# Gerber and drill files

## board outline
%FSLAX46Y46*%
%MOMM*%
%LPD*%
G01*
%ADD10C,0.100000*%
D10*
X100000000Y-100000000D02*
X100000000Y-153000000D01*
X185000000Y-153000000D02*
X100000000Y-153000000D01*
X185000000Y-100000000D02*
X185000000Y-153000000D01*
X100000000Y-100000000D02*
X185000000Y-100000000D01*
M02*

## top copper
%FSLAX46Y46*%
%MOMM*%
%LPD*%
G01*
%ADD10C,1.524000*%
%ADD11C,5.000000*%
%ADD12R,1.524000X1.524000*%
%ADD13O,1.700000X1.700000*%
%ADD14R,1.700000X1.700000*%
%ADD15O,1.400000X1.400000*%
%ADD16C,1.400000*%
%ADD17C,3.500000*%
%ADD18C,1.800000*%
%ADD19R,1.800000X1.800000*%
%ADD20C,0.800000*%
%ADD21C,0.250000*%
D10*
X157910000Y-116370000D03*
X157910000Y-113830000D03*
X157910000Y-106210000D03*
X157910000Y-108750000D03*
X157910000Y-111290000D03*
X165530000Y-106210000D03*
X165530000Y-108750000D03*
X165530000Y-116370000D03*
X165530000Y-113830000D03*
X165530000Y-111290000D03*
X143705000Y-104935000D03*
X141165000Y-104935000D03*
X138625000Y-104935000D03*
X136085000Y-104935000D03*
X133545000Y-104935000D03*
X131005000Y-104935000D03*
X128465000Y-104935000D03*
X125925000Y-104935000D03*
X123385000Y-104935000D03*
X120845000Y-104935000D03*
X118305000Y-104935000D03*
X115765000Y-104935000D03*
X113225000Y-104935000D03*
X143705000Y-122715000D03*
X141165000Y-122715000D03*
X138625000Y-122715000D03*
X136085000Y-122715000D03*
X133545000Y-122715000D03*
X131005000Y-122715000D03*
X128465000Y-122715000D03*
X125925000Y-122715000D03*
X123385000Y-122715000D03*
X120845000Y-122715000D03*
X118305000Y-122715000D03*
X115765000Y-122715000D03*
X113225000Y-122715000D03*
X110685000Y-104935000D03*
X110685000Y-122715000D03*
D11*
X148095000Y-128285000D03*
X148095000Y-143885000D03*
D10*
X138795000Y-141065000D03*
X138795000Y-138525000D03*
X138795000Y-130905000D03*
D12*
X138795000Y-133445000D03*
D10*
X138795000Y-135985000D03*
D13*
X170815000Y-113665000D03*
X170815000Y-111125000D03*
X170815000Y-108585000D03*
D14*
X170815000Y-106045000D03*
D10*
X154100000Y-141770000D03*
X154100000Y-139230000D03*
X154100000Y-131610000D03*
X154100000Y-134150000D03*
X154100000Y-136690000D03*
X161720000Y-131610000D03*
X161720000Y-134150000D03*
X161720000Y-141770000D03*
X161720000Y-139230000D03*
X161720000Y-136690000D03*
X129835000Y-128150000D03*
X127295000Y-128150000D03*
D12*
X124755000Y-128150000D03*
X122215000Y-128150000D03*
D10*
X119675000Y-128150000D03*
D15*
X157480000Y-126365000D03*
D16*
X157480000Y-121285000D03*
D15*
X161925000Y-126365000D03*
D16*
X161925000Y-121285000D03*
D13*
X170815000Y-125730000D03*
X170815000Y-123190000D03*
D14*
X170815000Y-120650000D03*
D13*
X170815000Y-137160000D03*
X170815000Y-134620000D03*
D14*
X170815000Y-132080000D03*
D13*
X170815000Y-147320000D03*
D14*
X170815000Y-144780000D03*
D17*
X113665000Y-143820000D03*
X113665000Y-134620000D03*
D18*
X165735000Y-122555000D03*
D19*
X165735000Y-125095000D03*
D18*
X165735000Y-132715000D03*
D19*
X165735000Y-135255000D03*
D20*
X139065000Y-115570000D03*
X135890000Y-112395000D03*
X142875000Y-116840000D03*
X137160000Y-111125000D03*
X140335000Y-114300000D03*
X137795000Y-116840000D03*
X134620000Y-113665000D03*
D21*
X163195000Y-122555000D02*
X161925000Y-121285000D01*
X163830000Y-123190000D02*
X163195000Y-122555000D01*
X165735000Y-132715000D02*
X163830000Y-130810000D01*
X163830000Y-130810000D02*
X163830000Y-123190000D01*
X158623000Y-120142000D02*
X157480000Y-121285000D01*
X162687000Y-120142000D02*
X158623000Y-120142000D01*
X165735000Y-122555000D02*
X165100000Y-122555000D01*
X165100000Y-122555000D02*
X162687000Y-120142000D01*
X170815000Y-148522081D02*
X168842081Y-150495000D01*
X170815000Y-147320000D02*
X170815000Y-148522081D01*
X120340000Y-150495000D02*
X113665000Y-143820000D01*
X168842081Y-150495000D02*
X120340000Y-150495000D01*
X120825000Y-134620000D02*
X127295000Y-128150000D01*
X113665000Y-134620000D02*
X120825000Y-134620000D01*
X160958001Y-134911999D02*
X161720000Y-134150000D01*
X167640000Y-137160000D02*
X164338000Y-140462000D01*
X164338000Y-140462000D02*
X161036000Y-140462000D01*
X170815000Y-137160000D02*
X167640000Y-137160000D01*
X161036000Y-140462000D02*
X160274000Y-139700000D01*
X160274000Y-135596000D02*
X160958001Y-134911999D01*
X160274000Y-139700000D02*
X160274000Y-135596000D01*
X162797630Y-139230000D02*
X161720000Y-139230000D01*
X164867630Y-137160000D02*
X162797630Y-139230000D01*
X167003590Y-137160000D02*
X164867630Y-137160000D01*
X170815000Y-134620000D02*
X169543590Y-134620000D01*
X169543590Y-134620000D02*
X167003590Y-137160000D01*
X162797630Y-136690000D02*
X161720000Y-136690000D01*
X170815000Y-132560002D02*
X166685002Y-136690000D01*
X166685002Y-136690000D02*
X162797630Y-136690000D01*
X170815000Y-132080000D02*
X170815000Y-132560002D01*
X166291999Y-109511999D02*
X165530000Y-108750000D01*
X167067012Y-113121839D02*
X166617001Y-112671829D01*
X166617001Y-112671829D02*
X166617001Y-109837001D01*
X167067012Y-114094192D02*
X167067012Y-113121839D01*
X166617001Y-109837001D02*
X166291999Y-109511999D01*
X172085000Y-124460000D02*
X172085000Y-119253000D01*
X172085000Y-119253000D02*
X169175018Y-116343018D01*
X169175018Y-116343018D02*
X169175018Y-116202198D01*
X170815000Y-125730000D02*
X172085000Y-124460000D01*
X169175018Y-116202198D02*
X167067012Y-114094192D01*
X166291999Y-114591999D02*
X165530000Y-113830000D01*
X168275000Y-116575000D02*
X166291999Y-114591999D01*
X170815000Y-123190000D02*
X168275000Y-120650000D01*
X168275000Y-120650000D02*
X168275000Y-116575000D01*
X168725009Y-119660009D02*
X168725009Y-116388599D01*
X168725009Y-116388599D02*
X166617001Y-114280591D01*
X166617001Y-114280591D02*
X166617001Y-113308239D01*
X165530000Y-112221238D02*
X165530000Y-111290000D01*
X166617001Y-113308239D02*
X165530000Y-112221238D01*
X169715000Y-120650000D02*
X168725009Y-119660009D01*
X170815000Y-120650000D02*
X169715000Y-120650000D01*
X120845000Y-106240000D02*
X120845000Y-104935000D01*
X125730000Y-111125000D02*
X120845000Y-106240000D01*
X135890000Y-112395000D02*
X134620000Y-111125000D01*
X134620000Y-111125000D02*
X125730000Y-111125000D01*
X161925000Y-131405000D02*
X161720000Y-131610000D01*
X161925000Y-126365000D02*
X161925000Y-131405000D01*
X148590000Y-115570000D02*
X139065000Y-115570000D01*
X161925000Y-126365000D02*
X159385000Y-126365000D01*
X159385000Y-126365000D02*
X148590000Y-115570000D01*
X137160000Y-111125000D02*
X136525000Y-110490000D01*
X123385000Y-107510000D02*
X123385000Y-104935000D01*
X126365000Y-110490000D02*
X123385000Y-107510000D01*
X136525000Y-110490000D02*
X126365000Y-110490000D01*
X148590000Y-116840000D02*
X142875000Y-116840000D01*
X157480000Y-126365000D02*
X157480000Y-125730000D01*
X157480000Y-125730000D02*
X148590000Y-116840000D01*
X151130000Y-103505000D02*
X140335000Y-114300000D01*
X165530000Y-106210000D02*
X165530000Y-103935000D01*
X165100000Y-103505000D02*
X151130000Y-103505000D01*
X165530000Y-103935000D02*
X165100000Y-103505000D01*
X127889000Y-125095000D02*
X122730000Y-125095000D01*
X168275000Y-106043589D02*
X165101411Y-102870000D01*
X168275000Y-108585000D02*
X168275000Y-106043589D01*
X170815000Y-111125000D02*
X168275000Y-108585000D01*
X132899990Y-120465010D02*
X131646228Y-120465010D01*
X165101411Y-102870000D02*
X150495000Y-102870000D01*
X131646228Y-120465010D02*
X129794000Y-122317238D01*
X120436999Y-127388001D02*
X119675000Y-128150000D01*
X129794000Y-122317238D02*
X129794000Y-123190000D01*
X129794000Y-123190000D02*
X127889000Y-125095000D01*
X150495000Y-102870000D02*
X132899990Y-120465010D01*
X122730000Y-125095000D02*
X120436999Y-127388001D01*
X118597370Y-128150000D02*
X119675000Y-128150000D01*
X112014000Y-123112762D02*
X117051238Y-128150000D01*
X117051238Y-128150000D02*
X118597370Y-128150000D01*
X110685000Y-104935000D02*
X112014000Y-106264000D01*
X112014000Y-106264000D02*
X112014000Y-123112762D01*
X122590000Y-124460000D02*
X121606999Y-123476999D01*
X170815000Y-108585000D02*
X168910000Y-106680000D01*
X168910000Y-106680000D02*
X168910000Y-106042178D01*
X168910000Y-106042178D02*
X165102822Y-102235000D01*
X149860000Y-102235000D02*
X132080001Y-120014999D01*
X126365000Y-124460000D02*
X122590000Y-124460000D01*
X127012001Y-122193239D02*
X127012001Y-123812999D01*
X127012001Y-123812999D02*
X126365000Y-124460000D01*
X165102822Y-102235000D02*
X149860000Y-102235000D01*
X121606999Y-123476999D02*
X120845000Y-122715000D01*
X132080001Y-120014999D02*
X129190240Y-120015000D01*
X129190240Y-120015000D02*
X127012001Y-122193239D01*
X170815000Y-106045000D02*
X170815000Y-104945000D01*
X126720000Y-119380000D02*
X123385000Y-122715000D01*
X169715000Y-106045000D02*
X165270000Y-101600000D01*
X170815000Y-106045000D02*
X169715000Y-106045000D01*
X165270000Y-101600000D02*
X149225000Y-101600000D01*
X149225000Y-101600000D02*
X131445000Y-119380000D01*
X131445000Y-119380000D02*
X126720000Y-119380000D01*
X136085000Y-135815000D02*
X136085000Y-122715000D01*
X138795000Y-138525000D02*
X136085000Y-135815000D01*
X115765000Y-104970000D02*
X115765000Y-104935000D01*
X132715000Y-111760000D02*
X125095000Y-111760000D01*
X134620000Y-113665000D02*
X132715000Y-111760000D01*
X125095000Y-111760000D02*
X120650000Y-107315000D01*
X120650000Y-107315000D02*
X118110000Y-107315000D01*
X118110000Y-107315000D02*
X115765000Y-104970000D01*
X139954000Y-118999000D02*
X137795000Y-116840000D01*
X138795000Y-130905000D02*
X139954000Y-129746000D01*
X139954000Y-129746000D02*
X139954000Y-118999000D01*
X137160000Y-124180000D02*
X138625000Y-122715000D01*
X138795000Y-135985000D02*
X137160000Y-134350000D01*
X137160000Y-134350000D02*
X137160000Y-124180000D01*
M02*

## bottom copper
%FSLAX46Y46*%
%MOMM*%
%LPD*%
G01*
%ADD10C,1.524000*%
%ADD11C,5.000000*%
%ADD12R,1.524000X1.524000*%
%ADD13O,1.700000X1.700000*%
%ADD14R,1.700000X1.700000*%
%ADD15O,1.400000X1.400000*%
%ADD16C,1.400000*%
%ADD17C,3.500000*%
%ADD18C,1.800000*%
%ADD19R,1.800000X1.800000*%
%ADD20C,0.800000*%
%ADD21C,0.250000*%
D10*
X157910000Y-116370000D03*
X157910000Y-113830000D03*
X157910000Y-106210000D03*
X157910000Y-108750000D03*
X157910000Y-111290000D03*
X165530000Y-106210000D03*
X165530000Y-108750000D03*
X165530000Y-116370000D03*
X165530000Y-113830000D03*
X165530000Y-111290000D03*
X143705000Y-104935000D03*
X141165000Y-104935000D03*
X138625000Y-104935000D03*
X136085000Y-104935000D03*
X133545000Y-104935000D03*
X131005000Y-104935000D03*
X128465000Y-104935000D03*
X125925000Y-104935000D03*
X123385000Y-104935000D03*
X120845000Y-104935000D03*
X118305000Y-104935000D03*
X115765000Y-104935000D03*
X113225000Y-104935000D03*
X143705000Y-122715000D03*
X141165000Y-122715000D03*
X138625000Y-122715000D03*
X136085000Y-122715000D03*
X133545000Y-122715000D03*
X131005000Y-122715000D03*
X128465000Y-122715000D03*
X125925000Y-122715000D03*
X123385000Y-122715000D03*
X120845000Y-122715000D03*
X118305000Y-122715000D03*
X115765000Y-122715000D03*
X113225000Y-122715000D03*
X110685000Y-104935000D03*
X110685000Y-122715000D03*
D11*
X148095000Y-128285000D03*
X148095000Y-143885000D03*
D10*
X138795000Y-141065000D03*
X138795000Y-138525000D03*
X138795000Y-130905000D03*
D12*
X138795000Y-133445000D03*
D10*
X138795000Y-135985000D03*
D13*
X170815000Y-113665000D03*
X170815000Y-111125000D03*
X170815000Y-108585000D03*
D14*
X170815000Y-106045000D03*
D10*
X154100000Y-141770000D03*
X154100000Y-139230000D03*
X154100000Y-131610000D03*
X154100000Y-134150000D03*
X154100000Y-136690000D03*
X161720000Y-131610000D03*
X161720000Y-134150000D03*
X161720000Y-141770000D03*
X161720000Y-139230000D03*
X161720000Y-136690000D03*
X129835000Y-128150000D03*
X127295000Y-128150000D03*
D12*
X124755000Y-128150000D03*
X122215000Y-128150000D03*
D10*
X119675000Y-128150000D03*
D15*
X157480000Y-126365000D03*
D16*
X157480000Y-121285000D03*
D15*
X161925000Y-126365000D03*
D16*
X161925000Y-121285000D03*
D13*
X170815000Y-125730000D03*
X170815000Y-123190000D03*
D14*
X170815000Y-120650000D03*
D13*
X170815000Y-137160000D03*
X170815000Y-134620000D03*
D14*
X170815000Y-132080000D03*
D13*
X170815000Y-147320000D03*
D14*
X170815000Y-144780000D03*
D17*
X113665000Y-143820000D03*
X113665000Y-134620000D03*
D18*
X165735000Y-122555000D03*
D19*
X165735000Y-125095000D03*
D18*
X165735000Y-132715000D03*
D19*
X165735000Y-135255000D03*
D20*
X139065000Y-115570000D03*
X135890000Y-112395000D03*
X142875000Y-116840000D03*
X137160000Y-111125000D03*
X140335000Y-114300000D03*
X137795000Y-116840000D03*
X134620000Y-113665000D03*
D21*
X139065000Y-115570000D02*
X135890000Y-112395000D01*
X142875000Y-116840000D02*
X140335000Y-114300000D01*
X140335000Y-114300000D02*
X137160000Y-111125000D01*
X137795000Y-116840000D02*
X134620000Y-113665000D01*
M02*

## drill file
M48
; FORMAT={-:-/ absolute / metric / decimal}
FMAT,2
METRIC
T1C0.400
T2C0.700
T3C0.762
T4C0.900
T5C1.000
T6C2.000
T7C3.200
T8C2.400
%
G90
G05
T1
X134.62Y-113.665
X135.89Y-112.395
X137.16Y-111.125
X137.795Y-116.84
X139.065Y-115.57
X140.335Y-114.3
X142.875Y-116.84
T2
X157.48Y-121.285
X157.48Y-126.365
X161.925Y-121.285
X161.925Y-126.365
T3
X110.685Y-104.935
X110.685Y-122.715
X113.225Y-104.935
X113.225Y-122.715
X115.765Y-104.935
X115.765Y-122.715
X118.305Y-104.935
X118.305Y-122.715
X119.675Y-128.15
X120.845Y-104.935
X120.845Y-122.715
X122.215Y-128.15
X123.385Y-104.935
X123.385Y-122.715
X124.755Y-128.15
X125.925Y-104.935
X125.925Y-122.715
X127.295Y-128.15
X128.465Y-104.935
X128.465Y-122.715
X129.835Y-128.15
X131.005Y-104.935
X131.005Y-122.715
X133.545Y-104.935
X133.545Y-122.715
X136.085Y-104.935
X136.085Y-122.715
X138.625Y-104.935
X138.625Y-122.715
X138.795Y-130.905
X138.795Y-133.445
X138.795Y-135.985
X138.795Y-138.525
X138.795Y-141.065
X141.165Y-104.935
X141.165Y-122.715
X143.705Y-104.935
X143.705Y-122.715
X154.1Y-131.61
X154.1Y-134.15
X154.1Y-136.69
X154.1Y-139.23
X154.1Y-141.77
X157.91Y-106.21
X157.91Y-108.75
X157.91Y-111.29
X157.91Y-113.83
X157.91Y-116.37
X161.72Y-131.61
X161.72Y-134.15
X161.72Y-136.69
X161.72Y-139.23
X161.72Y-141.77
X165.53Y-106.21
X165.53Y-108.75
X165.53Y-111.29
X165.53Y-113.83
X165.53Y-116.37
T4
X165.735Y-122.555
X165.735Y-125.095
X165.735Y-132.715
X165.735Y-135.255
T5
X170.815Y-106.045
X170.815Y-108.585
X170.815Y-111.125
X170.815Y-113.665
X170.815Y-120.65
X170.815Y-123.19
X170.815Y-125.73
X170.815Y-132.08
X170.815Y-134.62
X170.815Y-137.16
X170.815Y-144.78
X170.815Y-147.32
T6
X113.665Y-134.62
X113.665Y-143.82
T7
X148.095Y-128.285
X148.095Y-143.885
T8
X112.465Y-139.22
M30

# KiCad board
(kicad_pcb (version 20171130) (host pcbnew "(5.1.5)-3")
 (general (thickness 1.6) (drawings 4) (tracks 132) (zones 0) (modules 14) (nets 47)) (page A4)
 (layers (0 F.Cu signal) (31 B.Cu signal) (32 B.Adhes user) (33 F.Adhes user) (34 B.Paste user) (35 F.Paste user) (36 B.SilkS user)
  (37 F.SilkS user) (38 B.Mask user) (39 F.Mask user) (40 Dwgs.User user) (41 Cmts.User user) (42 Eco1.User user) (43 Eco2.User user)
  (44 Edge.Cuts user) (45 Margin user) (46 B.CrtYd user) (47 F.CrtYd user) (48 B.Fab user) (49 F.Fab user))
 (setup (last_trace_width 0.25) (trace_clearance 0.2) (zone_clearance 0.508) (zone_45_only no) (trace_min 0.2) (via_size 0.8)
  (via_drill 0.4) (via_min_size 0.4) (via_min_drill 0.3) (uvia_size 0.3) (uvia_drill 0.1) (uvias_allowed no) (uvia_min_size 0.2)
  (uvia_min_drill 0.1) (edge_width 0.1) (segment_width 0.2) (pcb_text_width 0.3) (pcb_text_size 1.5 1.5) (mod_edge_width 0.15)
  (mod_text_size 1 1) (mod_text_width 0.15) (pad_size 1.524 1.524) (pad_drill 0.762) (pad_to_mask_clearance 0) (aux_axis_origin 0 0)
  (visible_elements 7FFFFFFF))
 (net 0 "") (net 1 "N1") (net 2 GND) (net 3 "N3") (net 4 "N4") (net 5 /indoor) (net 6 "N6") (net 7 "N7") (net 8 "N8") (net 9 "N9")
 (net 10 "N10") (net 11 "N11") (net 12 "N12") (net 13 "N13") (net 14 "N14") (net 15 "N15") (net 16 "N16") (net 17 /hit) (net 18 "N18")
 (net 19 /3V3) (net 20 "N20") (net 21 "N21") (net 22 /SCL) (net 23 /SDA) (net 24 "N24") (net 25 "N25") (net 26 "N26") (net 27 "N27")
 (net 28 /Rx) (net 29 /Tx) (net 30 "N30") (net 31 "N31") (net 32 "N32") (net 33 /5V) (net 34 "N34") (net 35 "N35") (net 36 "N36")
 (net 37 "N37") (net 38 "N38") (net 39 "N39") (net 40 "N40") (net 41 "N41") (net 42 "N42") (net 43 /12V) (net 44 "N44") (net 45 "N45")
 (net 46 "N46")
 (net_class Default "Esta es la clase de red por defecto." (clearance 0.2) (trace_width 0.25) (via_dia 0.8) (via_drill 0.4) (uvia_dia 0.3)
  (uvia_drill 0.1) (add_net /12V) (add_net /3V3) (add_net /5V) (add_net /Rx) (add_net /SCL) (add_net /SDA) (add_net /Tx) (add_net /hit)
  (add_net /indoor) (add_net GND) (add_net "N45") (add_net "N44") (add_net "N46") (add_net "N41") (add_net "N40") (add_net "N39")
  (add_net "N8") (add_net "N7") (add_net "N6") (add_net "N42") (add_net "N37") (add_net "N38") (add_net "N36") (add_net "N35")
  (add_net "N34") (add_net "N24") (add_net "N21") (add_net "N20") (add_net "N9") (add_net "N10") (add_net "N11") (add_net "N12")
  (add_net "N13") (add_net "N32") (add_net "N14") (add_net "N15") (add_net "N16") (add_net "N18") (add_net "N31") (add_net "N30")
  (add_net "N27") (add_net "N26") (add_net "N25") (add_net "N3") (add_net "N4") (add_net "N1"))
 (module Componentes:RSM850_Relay (layer F.Cu) (at 166.37 104.14 270)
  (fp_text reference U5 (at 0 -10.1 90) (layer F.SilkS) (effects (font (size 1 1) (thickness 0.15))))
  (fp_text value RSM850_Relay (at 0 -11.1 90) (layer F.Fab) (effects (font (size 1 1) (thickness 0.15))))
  (pad "" thru_hole circle (at 12.23 8.46 270) (size 1.524 1.524) (drill 0.762) (layers *.Cu *.Mask))
  (pad 8 thru_hole circle (at 9.69 8.46 270) (size 1.524 1.524) (drill 0.762) (layers *.Cu *.Mask) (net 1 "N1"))
  (pad 2 thru_hole circle (at 2.07 8.46 270) (size 1.524 1.524) (drill 0.762) (layers *.Cu *.Mask) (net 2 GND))
  (pad 6 thru_hole circle (at 4.61 8.46 270) (size 1.524 1.524) (drill 0.762) (layers *.Cu *.Mask) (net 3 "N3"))
  (pad 7 thru_hole circle (at 7.15 8.46 270) (size 1.524 1.524) (drill 0.762) (layers *.Cu *.Mask) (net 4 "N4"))
  (pad 1 thru_hole circle (at 2.07 0.84 270) (size 1.524 1.524) (drill 0.762) (layers *.Cu *.Mask) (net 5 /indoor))
  (pad 3 thru_hole circle (at 4.61 0.84 270) (size 1.524 1.524) (drill 0.762) (layers *.Cu *.Mask) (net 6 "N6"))
  (pad "" thru_hole circle (at 12.23 0.84 270) (size 1.524 1.524) (drill 0.762) (layers *.Cu *.Mask))
  (pad 5 thru_hole circle (at 9.69 0.84 270) (size 1.524 1.524) (drill 0.762) (layers *.Cu *.Mask) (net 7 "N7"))
  (pad 4 thru_hole circle (at 7.15 0.84 270) (size 1.524 1.524) (drill 0.762) (layers *.Cu *.Mask) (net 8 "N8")))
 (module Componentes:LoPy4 (layer F.Cu) (at 100.965 123.825 90)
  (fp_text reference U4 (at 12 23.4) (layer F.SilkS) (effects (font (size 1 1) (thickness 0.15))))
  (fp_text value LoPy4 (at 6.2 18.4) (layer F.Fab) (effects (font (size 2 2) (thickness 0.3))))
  (pad 15 thru_hole circle (at 18.89 42.74 90) (size 1.524 1.524) (drill 0.762) (layers *.Cu *.Mask) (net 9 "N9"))
  (pad 16 thru_hole circle (at 18.89 40.2 90) (size 1.524 1.524) (drill 0.762) (layers *.Cu *.Mask) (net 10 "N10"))
  (pad 17 thru_hole circle (at 18.89 37.66 90) (size 1.524 1.524) (drill 0.762) (layers *.Cu *.Mask) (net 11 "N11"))
  (pad 18 thru_hole circle (at 18.89 35.12 90) (size 1.524 1.524) (drill 0.762) (layers *.Cu *.Mask) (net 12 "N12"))
  (pad 19 thru_hole circle (at 18.89 32.58 90) (size 1.524 1.524) (drill 0.762) (layers *.Cu *.Mask) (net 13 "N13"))
  (pad 20 thru_hole circle (at 18.89 30.04 90) (size 1.524 1.524) (drill 0.762) (layers *.Cu *.Mask) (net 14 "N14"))
  (pad 21 thru_hole circle (at 18.89 27.5 90) (size 1.524 1.524) (drill 0.762) (layers *.Cu *.Mask) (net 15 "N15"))
  (pad 22 thru_hole circle (at 18.89 24.96 90) (size 1.524 1.524) (drill 0.762) (layers *.Cu *.Mask) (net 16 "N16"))
  (pad 23 thru_hole circle (at 18.89 22.42 90) (size 1.524 1.524) (drill 0.762) (layers *.Cu *.Mask) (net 5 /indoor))
  (pad 24 thru_hole circle (at 18.89 19.88 90) (size 1.524 1.524) (drill 0.762) (layers *.Cu *.Mask) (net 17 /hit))
  (pad 25 thru_hole circle (at 18.89 17.34 90) (size 1.524 1.524) (drill 0.762) (layers *.Cu *.Mask) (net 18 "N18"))
  (pad 26 thru_hole circle (at 18.89 14.8 90) (size 1.524 1.524) (drill 0.762) (layers *.Cu *.Mask) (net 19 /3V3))
  (pad 27 thru_hole circle (at 18.89 12.26 90) (size 1.524 1.524) (drill 0.762) (layers *.Cu *.Mask) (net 2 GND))
  (pad 14 thru_hole circle (at 1.11 42.74 90) (size 1.524 1.524) (drill 0.762) (layers *.Cu *.Mask) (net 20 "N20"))
  (pad 13 thru_hole circle (at 1.11 40.2 90) (size 1.524 1.524) (drill 0.762) (layers *.Cu *.Mask) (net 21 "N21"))
  (pad 12 thru_hole circle (at 1.11 37.66 90) (size 1.524 1.524) (drill 0.762) (layers *.Cu *.Mask) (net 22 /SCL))
  (pad 11 thru_hole circle (at 1.11 35.12 90) (size 1.524 1.524) (drill 0.762) (layers *.Cu *.Mask) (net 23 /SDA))
  (pad 10 thru_hole circle (at 1.11 32.58 90) (size 1.524 1.524) (drill 0.762) (layers *.Cu *.Mask) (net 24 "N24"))
  (pad 9 thru_hole circle (at 1.11 30.04 90) (size 1.524 1.524) (drill 0.762) (layers *.Cu *.Mask) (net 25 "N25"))
  (pad 8 thru_hole circle (at 1.11 27.5 90) (size 1.524 1.524) (drill 0.762) (layers *.Cu *.Mask) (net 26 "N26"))
  (pad 7 thru_hole circle (at 1.11 24.96 90) (size 1.524 1.524) (drill 0.762) (layers *.Cu *.Mask) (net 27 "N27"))
  (pad 6 thru_hole circle (at 1.11 22.42 90) (size 1.524 1.524) (drill 0.762) (layers *.Cu *.Mask) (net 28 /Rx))
  (pad 5 thru_hole circle (at 1.11 19.88 90) (size 1.524 1.524) (drill 0.762) (layers *.Cu *.Mask) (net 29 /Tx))
  (pad 4 thru_hole circle (at 1.11 17.34 90) (size 1.524 1.524) (drill 0.762) (layers *.Cu *.Mask) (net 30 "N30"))
  (pad 3 thru_hole circle (at 1.11 14.8 90) (size 1.524 1.524) (drill 0.762) (layers *.Cu *.Mask) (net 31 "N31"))
  (pad 2 thru_hole circle (at 1.11 12.26 90) (size 1.524 1.524) (drill 0.762) (layers *.Cu *.Mask) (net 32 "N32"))
  (pad 28 thru_hole circle (at 18.89 9.72 90) (size 1.524 1.524) (drill 0.762) (layers *.Cu *.Mask) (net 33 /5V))
  (pad 1 thru_hole circle (at 1.11 9.72 90) (size 1.524 1.524) (drill 0.762) (layers *.Cu *.Mask) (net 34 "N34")))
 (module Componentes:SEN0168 (layer F.Cu) (at 137.795 146.685 90)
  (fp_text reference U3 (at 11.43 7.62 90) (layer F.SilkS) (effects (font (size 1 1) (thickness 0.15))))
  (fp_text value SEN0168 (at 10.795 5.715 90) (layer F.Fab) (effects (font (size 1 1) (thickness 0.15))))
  (pad "" thru_hole circle (at 18.4 10.3 90) (size 5 5) (drill 3.2) (layers *.Cu *.Mask))
  (pad "" thru_hole circle (at 2.8 10.3 90) (size 5 5) (drill 3.2) (layers *.Cu *.Mask))
  (pad 5 thru_hole circle (at 5.62 1 90) (size 1.524 1.524) (drill 0.762) (layers *.Cu *.Mask) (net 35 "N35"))
  (pad 4 thru_hole circle (at 8.16 1 90) (size 1.524 1.524) (drill 0.762) (layers *.Cu *.Mask) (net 23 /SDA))
  (pad 1 thru_hole circle (at 15.78 1 90) (size 1.524 1.524) (drill 0.762) (layers *.Cu *.Mask) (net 19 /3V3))
  (pad 2 thru_hole rect (at 13.24 1 90) (size 1.524 1.524) (drill 0.762) (layers *.Cu *.Mask) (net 2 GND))
  (pad 3 thru_hole circle (at 10.7 1 90) (size 1.524 1.524) (drill 0.762) (layers *.Cu *.Mask) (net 22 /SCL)))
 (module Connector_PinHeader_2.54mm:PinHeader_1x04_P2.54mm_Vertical (layer F.Cu) (at 170.815 106.045)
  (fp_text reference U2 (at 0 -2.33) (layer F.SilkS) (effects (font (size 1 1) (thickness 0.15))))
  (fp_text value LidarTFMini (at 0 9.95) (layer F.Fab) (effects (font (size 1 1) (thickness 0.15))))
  (pad 4 thru_hole oval (at 0 7.62) (size 1.7 1.7) (drill 1) (layers *.Cu *.Mask) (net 2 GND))
  (pad 3 thru_hole oval (at 0 5.08) (size 1.7 1.7) (drill 1) (layers *.Cu *.Mask) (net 33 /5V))
  (pad 2 thru_hole oval (at 0 2.54) (size 1.7 1.7) (drill 1) (layers *.Cu *.Mask) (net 29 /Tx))
  (pad 1 thru_hole rect (at 0 0) (size 1.7 1.7) (drill 1) (layers *.Cu *.Mask) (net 28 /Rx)))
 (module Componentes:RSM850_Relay (layer F.Cu) (at 162.56 129.54 270)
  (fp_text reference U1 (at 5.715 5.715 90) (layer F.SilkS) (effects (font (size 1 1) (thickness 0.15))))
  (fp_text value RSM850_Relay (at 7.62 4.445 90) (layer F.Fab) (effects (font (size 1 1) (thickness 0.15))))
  (pad "" thru_hole circle (at 12.23 8.46 270) (size 1.524 1.524) (drill 0.762) (layers *.Cu *.Mask))
  (pad 8 thru_hole circle (at 9.69 8.46 270) (size 1.524 1.524) (drill 0.762) (layers *.Cu *.Mask) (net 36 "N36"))
  (pad 2 thru_hole circle (at 2.07 8.46 270) (size 1.524 1.524) (drill 0.762) (layers *.Cu *.Mask) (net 2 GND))
  (pad 6 thru_hole circle (at 4.61 8.46 270) (size 1.524 1.524) (drill 0.762) (layers *.Cu *.Mask) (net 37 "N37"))
  (pad 7 thru_hole circle (at 7.15 8.46 270) (size 1.524 1.524) (drill 0.762) (layers *.Cu *.Mask) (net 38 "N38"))
  (pad 1 thru_hole circle (at 2.07 0.84 270) (size 1.524 1.524) (drill 0.762) (layers *.Cu *.Mask) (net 17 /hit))
  (pad 3 thru_hole circle (at 4.61 0.84 270) (size 1.524 1.524) (drill 0.762) (layers *.Cu *.Mask) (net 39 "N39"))
  (pad "" thru_hole circle (at 12.23 0.84 270) (size 1.524 1.524) (drill 0.762) (layers *.Cu *.Mask))
  (pad 5 thru_hole circle (at 9.69 0.84 270) (size 1.524 1.524) (drill 0.762) (layers *.Cu *.Mask) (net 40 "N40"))
  (pad 4 thru_hole circle (at 7.15 0.84 270) (size 1.524 1.524) (drill 0.762) (layers *.Cu *.Mask) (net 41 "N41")))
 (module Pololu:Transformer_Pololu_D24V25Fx (layer F.Cu) (at 126.365 132.08)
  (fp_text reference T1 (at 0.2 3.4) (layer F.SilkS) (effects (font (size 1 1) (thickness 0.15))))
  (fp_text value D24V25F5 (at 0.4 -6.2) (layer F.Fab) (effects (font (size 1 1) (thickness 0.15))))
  (pad 3 thru_hole circle (at 3.47 -3.93) (size 1.524 1.524) (drill 0.762) (layers *.Cu *.Mask) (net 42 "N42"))
  (pad 1 thru_hole circle (at 0.93 -3.93) (size 1.524 1.524) (drill 0.762) (layers *.Cu *.Mask) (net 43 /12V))
  (pad 2 thru_hole rect (at -1.61 -3.93) (size 1.524 1.524) (drill 0.762) (layers *.Cu *.Mask) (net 2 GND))
  (pad 2 thru_hole rect (at -4.15 -3.93) (size 1.524 1.524) (drill 0.762) (layers *.Cu *.Mask) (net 2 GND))
  (pad 4 thru_hole circle (at -6.69 -3.93) (size 1.524 1.524) (drill 0.762) (layers *.Cu *.Mask) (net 33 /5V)))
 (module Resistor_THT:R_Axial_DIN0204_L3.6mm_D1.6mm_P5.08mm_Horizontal (layer F.Cu) (at 157.48 121.285 270)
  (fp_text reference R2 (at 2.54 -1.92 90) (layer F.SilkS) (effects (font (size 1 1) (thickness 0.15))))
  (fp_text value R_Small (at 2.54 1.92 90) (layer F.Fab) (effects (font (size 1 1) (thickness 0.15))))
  (pad 2 thru_hole oval (at 5.08 0 270) (size 1.4 1.4) (drill 0.7) (layers *.Cu *.Mask) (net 5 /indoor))
  (pad 1 thru_hole circle (at 0 0 270) (size 1.4 1.4) (drill 0.7) (layers *.Cu *.Mask) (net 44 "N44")))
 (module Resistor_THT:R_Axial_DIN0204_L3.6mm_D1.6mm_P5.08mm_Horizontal (layer F.Cu) (at 161.925 121.285 270)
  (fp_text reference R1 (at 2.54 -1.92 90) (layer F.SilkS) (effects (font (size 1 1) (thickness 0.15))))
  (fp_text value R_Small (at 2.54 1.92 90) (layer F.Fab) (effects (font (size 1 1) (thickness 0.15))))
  (pad 2 thru_hole oval (at 5.08 0 270) (size 1.4 1.4) (drill 0.7) (layers *.Cu *.Mask) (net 17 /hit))
  (pad 1 thru_hole circle (at 0 0 270) (size 1.4 1.4) (drill 0.7) (layers *.Cu *.Mask) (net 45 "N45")))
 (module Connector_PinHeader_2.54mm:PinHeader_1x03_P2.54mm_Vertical (layer F.Cu) (at 170.815 120.65)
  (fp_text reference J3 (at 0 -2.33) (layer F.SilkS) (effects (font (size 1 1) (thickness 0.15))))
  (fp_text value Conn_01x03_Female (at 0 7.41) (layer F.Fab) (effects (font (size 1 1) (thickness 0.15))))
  (pad 3 thru_hole oval (at 0 5.08) (size 1.7 1.7) (drill 1) (layers *.Cu *.Mask) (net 6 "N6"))
  (pad 2 thru_hole oval (at 0 2.54) (size 1.7 1.7) (drill 1) (layers *.Cu *.Mask) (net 7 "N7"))
  (pad 1 thru_hole rect (at 0 0) (size 1.7 1.7) (drill 1) (layers *.Cu *.Mask) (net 8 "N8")))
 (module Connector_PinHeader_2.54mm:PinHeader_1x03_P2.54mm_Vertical (layer F.Cu) (at 170.815 132.08)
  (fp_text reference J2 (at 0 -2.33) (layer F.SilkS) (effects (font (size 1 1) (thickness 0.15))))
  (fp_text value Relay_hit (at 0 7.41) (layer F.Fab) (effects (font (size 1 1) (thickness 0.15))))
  (pad 3 thru_hole oval (at 0 5.08) (size 1.7 1.7) (drill 1) (layers *.Cu *.Mask) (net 39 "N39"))
  (pad 2 thru_hole oval (at 0 2.54) (size 1.7 1.7) (drill 1) (layers *.Cu *.Mask) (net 40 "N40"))
  (pad 1 thru_hole rect (at 0 0) (size 1.7 1.7) (drill 1) (layers *.Cu *.Mask) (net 41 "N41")))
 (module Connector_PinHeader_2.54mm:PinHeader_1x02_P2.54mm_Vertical (layer F.Cu) (at 170.815 144.78)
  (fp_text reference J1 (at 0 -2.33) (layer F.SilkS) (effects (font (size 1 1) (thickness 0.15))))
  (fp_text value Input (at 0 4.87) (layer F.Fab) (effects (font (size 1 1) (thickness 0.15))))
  (pad 2 thru_hole oval (at 0 2.54) (size 1.7 1.7) (drill 1) (layers *.Cu *.Mask) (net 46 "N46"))
  (pad 1 thru_hole rect (at 0 0) (size 1.7 1.7) (drill 1) (layers *.Cu *.Mask) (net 2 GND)))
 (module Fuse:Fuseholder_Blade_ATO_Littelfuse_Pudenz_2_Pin (layer F.Cu) (at 113.665 134.62 270)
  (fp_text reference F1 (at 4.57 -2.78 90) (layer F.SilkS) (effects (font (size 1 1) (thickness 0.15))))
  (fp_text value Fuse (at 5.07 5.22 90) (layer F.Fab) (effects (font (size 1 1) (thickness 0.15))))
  (pad 2 thru_hole circle (at 9.2 0 270) (size 3.5 3.5) (drill 2) (layers *.Cu *.Mask) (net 46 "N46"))
  (pad "" np_thru_hole circle (at 4.6 1.2 270) (size 2.4 2.4) (drill 2.4) (layers *.Cu *.Mask))
  (pad 1 thru_hole circle (at 0 0 270) (size 3.5 3.5) (drill 2) (layers *.Cu *.Mask) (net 43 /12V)))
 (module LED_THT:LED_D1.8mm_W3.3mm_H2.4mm (layer F.Cu) (at 165.735 125.095 90)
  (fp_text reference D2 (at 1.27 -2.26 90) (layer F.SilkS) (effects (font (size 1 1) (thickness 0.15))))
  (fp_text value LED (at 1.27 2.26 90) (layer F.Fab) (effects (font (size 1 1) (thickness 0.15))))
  (pad 2 thru_hole circle (at 2.54 0 90) (size 1.8 1.8) (drill 0.9) (layers *.Cu *.Mask) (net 44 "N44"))
  (pad 1 thru_hole rect (at 0 0 90) (size 1.8 1.8) (drill 0.9) (layers *.Cu *.Mask) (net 2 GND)))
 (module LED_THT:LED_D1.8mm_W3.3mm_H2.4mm (layer F.Cu) (at 165.735 135.255 90)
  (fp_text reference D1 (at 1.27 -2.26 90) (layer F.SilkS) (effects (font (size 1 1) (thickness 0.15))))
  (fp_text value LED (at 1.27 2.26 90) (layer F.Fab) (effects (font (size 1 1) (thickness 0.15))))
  (pad 2 thru_hole circle (at 2.54 0 90) (size 1.8 1.8) (drill 0.9) (layers *.Cu *.Mask) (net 45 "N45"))
  (pad 1 thru_hole rect (at 0 0 90) (size 1.8 1.8) (drill 0.9) (layers *.Cu *.Mask) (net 2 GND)))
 (gr_line (start 100 100) (end 100 153) (layer Edge.Cuts) (width 0.1))
 (gr_line (start 185 153) (end 100 153) (layer Edge.Cuts) (width 0.1))
 (gr_line (start 185 100) (end 185 153) (layer Edge.Cuts) (width 0.1))
 (gr_line (start 100 100) (end 185 100) (layer Edge.Cuts) (width 0.1))
 (segment (start 163.195 122.555) (end 161.925 121.285) (width 0.25) (layer F.Cu) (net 45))
 (segment (start 163.83 123.19) (end 163.195 122.555) (width 0.25) (layer F.Cu) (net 45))
 (segment (start 165.735 132.715) (end 163.83 130.81) (width 0.25) (layer F.Cu) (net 45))
 (segment (start 163.83 130.81) (end 163.83 123.19) (width 0.25) (layer F.Cu) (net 45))
 (segment (start 158.623 120.142) (end 157.48 121.285) (width 0.25) (layer F.Cu) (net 44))
 (segment (start 162.687 120.142) (end 158.623 120.142) (width 0.25) (layer F.Cu) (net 44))
 (segment (start 165.735 122.555) (end 165.1 122.555) (width 0.25) (layer F.Cu) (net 44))
 (segment (start 165.1 122.555) (end 162.687 120.142) (width 0.25) (layer F.Cu) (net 44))
 (segment (start 170.815 148.522081) (end 168.842081 150.495) (width 0.25) (layer F.Cu) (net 46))
 (segment (start 170.815 147.32) (end 170.815 148.522081) (width 0.25) (layer F.Cu) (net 46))
 (segment (start 120.34 150.495) (end 113.665 143.82) (width 0.25) (layer F.Cu) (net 46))
 (segment (start 168.842081 150.495) (end 120.34 150.495) (width 0.25) (layer F.Cu) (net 46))
 (segment (start 120.825 134.62) (end 127.295 128.15) (width 0.25) (layer F.Cu) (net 43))
 (segment (start 113.665 134.62) (end 120.825 134.62) (width 0.25) (layer F.Cu) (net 43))
 (segment (start 160.958001 134.911999) (end 161.72 134.15) (width 0.25) (layer F.Cu) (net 39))
 (segment (start 167.64 137.16) (end 164.338 140.462) (width 0.25) (layer F.Cu) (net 39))
 (segment (start 164.338 140.462) (end 161.036 140.462) (width 0.25) (layer F.Cu) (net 39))
 (segment (start 170.815 137.16) (end 167.64 137.16) (width 0.25) (layer F.Cu) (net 39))
 (segment (start 161.036 140.462) (end 160.274 139.7) (width 0.25) (layer F.Cu) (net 39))
 (segment (start 160.274 135.596) (end 160.958001 134.911999) (width 0.25) (layer F.Cu) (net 39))
 (segment (start 160.274 139.7) (end 160.274 135.596) (width 0.25) (layer F.Cu) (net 39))
 (segment (start 162.79763 139.23) (end 161.72 139.23) (width 0.25) (layer F.Cu) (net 40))
 (segment (start 164.86763 137.16) (end 162.79763 139.23) (width 0.25) (layer F.Cu) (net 40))
 (segment (start 167.00359 137.16) (end 164.86763 137.16) (width 0.25) (layer F.Cu) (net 40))
 (segment (start 170.815 134.62) (end 169.54359 134.62) (width 0.25) (layer F.Cu) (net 40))
 (segment (start 169.54359 134.62) (end 167.00359 137.16) (width 0.25) (layer F.Cu) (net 40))
 (segment (start 162.79763 136.69) (end 161.72 136.69) (width 0.25) (layer F.Cu) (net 41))
 (segment (start 170.815 132.560002) (end 166.685002 136.69) (width 0.25) (layer F.Cu) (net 41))
 (segment (start 166.685002 136.69) (end 162.79763 136.69) (width 0.25) (layer F.Cu) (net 41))
 (segment (start 170.815 132.08) (end 170.815 132.560002) (width 0.25) (layer F.Cu) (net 41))
 (segment (start 166.291999 109.511999) (end 165.53 108.75) (width 0.25) (layer F.Cu) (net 6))
 (segment (start 167.067012 113.121839) (end 166.617001 112.671829) (width 0.25) (layer F.Cu) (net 6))
 (segment (start 166.617001 112.671829) (end 166.617001 109.837001) (width 0.25) (layer F.Cu) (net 6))
 (segment (start 167.067012 114.094192) (end 167.067012 113.121839) (width 0.25) (layer F.Cu) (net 6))
 (segment (start 166.617001 109.837001) (end 166.291999 109.511999) (width 0.25) (layer F.Cu) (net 6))
 (segment (start 172.085 124.46) (end 172.085 119.253) (width 0.25) (layer F.Cu) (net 6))
 (segment (start 172.085 119.253) (end 169.175018 116.343018) (width 0.25) (layer F.Cu) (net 6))
 (segment (start 169.175018 116.343018) (end 169.175018 116.202198) (width 0.25) (layer F.Cu) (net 6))
 (segment (start 170.815 125.73) (end 172.085 124.46) (width 0.25) (layer F.Cu) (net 6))
 (segment (start 169.175018 116.202198) (end 167.067012 114.094192) (width 0.25) (layer F.Cu) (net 6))
 (segment (start 166.291999 114.591999) (end 165.53 113.83) (width 0.25) (layer F.Cu) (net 7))
 (segment (start 168.275 116.575) (end 166.291999 114.591999) (width 0.25) (layer F.Cu) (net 7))
 (segment (start 170.815 123.19) (end 168.275 120.65) (width 0.25) (layer F.Cu) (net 7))
 (segment (start 168.275 120.65) (end 168.275 116.575) (width 0.25) (layer F.Cu) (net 7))
 (segment (start 168.725009 119.660009) (end 168.725009 116.388599) (width 0.25) (layer F.Cu) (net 8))
 (segment (start 168.725009 116.388599) (end 166.617001 114.280591) (width 0.25) (layer F.Cu) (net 8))
 (segment (start 166.617001 114.280591) (end 166.617001 113.308239) (width 0.25) (layer F.Cu) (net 8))
 (segment (start 165.53 112.221238) (end 165.53 111.29) (width 0.25) (layer F.Cu) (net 8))
 (segment (start 166.617001 113.308239) (end 165.53 112.221238) (width 0.25) (layer F.Cu) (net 8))
 (segment (start 169.715 120.65) (end 168.725009 119.660009) (width 0.25) (layer F.Cu) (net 8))
 (segment (start 170.815 120.65) (end 169.715 120.65) (width 0.25) (layer F.Cu) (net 8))
 (via (at 139.065 115.57) (size 0.8) (drill 0.4) (layers F.Cu B.Cu) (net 17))
 (via (at 135.89 112.395) (size 0.8) (drill 0.4) (layers F.Cu B.Cu) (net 17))
 (segment (start 139.065 115.57) (end 135.89 112.395) (width 0.25) (layer B.Cu) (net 17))
 (segment (start 120.845 106.24) (end 120.845 104.935) (width 0.25) (layer F.Cu) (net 17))
 (segment (start 125.73 111.125) (end 120.845 106.24) (width 0.25) (layer F.Cu) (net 17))
 (segment (start 135.89 112.395) (end 134.62 111.125) (width 0.25) (layer F.Cu) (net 17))
 (segment (start 134.62 111.125) (end 125.73 111.125) (width 0.25) (layer F.Cu) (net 17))
 (segment (start 161.925 131.405) (end 161.72 131.61) (width 0.25) (layer F.Cu) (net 17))
 (segment (start 161.925 126.365) (end 161.925 131.405) (width 0.25) (layer F.Cu) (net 17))
 (segment (start 148.59 115.57) (end 139.065 115.57) (width 0.25) (layer F.Cu) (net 17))
 (segment (start 161.925 126.365) (end 159.385 126.365) (width 0.25) (layer F.Cu) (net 17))
 (segment (start 159.385 126.365) (end 148.59 115.57) (width 0.25) (layer F.Cu) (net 17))
 (via (at 142.875 116.84) (size 0.8) (drill 0.4) (layers F.Cu B.Cu) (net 5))
 (via (at 137.16 111.125) (size 0.8) (drill 0.4) (layers F.Cu B.Cu) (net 5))
 (segment (start 137.16 111.125) (end 136.525 110.49) (width 0.25) (layer F.Cu) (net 5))
 (segment (start 123.385 107.51) (end 123.385 104.935) (width 0.25) (layer F.Cu) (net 5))
 (segment (start 126.365 110.49) (end 123.385 107.51) (width 0.25) (layer F.Cu) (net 5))
 (segment (start 136.525 110.49) (end 126.365 110.49) (width 0.25) (layer F.Cu) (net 5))
 (segment (start 148.59 116.84) (end 142.875 116.84) (width 0.25) (layer F.Cu) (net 5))
 (segment (start 157.48 126.365) (end 157.48 125.73) (width 0.25) (layer F.Cu) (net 5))
 (segment (start 157.48 125.73) (end 148.59 116.84) (width 0.25) (layer F.Cu) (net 5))
 (via (at 140.335 114.3) (size 0.8) (drill 0.4) (layers F.Cu B.Cu) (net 5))
 (segment (start 142.875 116.84) (end 140.335 114.3) (width 0.25) (layer B.Cu) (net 5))
 (segment (start 140.335 114.3) (end 137.16 111.125) (width 0.25) (layer B.Cu) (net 5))
 (segment (start 151.13 103.505) (end 140.335 114.3) (width 0.25) (layer F.Cu) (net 5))
 (segment (start 165.53 106.21) (end 165.53 103.935) (width 0.25) (layer F.Cu) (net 5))
 (segment (start 165.1 103.505) (end 151.13 103.505) (width 0.25) (layer F.Cu) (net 5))
 (segment (start 165.53 103.935) (end 165.1 103.505) (width 0.25) (layer F.Cu) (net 5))
 (segment (start 127.889 125.095) (end 122.73 125.095) (width 0.25) (layer F.Cu) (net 33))
 (segment (start 168.275 106.043589) (end 165.101411 102.87) (width 0.25) (layer F.Cu) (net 33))
 (segment (start 168.275 108.585) (end 168.275 106.043589) (width 0.25) (layer F.Cu) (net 33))
 (segment (start 170.815 111.125) (end 168.275 108.585) (width 0.25) (layer F.Cu) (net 33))
 (segment (start 132.89999 120.46501) (end 131.646228 120.46501) (width 0.25) (layer F.Cu) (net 33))
 (segment (start 165.101411 102.87) (end 150.495 102.87) (width 0.25) (layer F.Cu) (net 33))
 (segment (start 131.646228 120.46501) (end 129.794 122.317238) (width 0.25) (layer F.Cu) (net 33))
 (segment (start 120.436999 127.388001) (end 119.675 128.15) (width 0.25) (layer F.Cu) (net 33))
 (segment (start 129.794 122.317238) (end 129.794 123.19) (width 0.25) (layer F.Cu) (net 33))
 (segment (start 129.794 123.19) (end 127.889 125.095) (width 0.25) (layer F.Cu) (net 33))
 (segment (start 150.495 102.87) (end 132.89999 120.46501) (width 0.25) (layer F.Cu) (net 33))
 (segment (start 122.73 125.095) (end 120.436999 127.388001) (width 0.25) (layer F.Cu) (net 33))
 (segment (start 118.59737 128.15) (end 119.675 128.15) (width 0.25) (layer F.Cu) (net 33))
 (segment (start 112.014 123.112762) (end 117.051238 128.15) (width 0.25) (layer F.Cu) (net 33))
 (segment (start 117.051238 128.15) (end 118.59737 128.15) (width 0.25) (layer F.Cu) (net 33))
 (segment (start 110.685 104.935) (end 112.014 106.264) (width 0.25) (layer F.Cu) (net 33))
 (segment (start 112.014 106.264) (end 112.014 123.112762) (width 0.25) (layer F.Cu) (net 33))
 (segment (start 122.59 124.46) (end 121.606999 123.476999) (width 0.25) (layer F.Cu) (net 29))
 (segment (start 170.815 108.585) (end 168.91 106.68) (width 0.25) (layer F.Cu) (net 29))
 (segment (start 168.91 106.68) (end 168.91 106.042178) (width 0.25) (layer F.Cu) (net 29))
 (segment (start 168.91 106.042178) (end 165.102822 102.235) (width 0.25) (layer F.Cu) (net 29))
 (segment (start 149.86 102.235) (end 132.080001 120.014999) (width 0.25) (layer F.Cu) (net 29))
 (segment (start 126.365 124.46) (end 122.59 124.46) (width 0.25) (layer F.Cu) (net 29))
 (segment (start 127.012001 122.193239) (end 127.012001 123.812999) (width 0.25) (layer F.Cu) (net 29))
 (segment (start 127.012001 123.812999) (end 126.365 124.46) (width 0.25) (layer F.Cu) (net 29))
 (segment (start 165.102822 102.235) (end 149.86 102.235) (width 0.25) (layer F.Cu) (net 29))
 (segment (start 121.606999 123.476999) (end 120.845 122.715) (width 0.25) (layer F.Cu) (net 29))
 (segment (start 132.080001 120.014999) (end 129.19024 120.015) (width 0.25) (layer F.Cu) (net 29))
 (segment (start 129.19024 120.015) (end 127.012001 122.193239) (width 0.25) (layer F.Cu) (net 29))
 (segment (start 170.815 106.045) (end 170.815 104.945) (width 0.25) (layer F.Cu) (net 28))
 (segment (start 126.72 119.38) (end 123.385 122.715) (width 0.25) (layer F.Cu) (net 28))
 (segment (start 169.715 106.045) (end 165.27 101.6) (width 0.25) (layer F.Cu) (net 28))
 (segment (start 170.815 106.045) (end 169.715 106.045) (width 0.25) (layer F.Cu) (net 28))
 (segment (start 165.27 101.6) (end 149.225 101.6) (width 0.25) (layer F.Cu) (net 28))
 (segment (start 149.225 101.6) (end 131.445 119.38) (width 0.25) (layer F.Cu) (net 28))
 (segment (start 131.445 119.38) (end 126.72 119.38) (width 0.25) (layer F.Cu) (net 28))
 (segment (start 136.085 135.815) (end 136.085 122.715) (width 0.25) (layer F.Cu) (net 23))
 (segment (start 138.795 138.525) (end 136.085 135.815) (width 0.25) (layer F.Cu) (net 23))
 (via (at 137.795 116.84) (size 0.8) (drill 0.4) (layers F.Cu B.Cu) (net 19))
 (via (at 134.62 113.665) (size 0.8) (drill 0.4) (layers F.Cu B.Cu) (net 19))
 (segment (start 137.795 116.84) (end 134.62 113.665) (width 0.25) (layer B.Cu) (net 19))
 (segment (start 115.765 104.97) (end 115.765 104.935) (width 0.25) (layer F.Cu) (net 19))
 (segment (start 132.715 111.76) (end 125.095 111.76) (width 0.25) (layer F.Cu) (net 19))
 (segment (start 134.62 113.665) (end 132.715 111.76) (width 0.25) (layer F.Cu) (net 19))
 (segment (start 125.095 111.76) (end 120.65 107.315) (width 0.25) (layer F.Cu) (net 19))
 (segment (start 120.65 107.315) (end 118.11 107.315) (width 0.25) (layer F.Cu) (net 19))
 (segment (start 118.11 107.315) (end 115.765 104.97) (width 0.25) (layer F.Cu) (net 19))
 (segment (start 139.954 118.999) (end 137.795 116.84) (width 0.25) (layer F.Cu) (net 19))
 (segment (start 138.795 130.905) (end 139.954 129.746) (width 0.25) (layer F.Cu) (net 19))
 (segment (start 139.954 129.746) (end 139.954 118.999) (width 0.25) (layer F.Cu) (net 19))
 (segment (start 137.16 124.18) (end 138.625 122.715) (width 0.25) (layer F.Cu) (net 22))
 (segment (start 138.795 135.985) (end 137.16 134.35) (width 0.25) (layer F.Cu) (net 22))
 (segment (start 137.16 134.35) (end 137.16 124.18) (width 0.25) (layer F.Cu) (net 22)))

